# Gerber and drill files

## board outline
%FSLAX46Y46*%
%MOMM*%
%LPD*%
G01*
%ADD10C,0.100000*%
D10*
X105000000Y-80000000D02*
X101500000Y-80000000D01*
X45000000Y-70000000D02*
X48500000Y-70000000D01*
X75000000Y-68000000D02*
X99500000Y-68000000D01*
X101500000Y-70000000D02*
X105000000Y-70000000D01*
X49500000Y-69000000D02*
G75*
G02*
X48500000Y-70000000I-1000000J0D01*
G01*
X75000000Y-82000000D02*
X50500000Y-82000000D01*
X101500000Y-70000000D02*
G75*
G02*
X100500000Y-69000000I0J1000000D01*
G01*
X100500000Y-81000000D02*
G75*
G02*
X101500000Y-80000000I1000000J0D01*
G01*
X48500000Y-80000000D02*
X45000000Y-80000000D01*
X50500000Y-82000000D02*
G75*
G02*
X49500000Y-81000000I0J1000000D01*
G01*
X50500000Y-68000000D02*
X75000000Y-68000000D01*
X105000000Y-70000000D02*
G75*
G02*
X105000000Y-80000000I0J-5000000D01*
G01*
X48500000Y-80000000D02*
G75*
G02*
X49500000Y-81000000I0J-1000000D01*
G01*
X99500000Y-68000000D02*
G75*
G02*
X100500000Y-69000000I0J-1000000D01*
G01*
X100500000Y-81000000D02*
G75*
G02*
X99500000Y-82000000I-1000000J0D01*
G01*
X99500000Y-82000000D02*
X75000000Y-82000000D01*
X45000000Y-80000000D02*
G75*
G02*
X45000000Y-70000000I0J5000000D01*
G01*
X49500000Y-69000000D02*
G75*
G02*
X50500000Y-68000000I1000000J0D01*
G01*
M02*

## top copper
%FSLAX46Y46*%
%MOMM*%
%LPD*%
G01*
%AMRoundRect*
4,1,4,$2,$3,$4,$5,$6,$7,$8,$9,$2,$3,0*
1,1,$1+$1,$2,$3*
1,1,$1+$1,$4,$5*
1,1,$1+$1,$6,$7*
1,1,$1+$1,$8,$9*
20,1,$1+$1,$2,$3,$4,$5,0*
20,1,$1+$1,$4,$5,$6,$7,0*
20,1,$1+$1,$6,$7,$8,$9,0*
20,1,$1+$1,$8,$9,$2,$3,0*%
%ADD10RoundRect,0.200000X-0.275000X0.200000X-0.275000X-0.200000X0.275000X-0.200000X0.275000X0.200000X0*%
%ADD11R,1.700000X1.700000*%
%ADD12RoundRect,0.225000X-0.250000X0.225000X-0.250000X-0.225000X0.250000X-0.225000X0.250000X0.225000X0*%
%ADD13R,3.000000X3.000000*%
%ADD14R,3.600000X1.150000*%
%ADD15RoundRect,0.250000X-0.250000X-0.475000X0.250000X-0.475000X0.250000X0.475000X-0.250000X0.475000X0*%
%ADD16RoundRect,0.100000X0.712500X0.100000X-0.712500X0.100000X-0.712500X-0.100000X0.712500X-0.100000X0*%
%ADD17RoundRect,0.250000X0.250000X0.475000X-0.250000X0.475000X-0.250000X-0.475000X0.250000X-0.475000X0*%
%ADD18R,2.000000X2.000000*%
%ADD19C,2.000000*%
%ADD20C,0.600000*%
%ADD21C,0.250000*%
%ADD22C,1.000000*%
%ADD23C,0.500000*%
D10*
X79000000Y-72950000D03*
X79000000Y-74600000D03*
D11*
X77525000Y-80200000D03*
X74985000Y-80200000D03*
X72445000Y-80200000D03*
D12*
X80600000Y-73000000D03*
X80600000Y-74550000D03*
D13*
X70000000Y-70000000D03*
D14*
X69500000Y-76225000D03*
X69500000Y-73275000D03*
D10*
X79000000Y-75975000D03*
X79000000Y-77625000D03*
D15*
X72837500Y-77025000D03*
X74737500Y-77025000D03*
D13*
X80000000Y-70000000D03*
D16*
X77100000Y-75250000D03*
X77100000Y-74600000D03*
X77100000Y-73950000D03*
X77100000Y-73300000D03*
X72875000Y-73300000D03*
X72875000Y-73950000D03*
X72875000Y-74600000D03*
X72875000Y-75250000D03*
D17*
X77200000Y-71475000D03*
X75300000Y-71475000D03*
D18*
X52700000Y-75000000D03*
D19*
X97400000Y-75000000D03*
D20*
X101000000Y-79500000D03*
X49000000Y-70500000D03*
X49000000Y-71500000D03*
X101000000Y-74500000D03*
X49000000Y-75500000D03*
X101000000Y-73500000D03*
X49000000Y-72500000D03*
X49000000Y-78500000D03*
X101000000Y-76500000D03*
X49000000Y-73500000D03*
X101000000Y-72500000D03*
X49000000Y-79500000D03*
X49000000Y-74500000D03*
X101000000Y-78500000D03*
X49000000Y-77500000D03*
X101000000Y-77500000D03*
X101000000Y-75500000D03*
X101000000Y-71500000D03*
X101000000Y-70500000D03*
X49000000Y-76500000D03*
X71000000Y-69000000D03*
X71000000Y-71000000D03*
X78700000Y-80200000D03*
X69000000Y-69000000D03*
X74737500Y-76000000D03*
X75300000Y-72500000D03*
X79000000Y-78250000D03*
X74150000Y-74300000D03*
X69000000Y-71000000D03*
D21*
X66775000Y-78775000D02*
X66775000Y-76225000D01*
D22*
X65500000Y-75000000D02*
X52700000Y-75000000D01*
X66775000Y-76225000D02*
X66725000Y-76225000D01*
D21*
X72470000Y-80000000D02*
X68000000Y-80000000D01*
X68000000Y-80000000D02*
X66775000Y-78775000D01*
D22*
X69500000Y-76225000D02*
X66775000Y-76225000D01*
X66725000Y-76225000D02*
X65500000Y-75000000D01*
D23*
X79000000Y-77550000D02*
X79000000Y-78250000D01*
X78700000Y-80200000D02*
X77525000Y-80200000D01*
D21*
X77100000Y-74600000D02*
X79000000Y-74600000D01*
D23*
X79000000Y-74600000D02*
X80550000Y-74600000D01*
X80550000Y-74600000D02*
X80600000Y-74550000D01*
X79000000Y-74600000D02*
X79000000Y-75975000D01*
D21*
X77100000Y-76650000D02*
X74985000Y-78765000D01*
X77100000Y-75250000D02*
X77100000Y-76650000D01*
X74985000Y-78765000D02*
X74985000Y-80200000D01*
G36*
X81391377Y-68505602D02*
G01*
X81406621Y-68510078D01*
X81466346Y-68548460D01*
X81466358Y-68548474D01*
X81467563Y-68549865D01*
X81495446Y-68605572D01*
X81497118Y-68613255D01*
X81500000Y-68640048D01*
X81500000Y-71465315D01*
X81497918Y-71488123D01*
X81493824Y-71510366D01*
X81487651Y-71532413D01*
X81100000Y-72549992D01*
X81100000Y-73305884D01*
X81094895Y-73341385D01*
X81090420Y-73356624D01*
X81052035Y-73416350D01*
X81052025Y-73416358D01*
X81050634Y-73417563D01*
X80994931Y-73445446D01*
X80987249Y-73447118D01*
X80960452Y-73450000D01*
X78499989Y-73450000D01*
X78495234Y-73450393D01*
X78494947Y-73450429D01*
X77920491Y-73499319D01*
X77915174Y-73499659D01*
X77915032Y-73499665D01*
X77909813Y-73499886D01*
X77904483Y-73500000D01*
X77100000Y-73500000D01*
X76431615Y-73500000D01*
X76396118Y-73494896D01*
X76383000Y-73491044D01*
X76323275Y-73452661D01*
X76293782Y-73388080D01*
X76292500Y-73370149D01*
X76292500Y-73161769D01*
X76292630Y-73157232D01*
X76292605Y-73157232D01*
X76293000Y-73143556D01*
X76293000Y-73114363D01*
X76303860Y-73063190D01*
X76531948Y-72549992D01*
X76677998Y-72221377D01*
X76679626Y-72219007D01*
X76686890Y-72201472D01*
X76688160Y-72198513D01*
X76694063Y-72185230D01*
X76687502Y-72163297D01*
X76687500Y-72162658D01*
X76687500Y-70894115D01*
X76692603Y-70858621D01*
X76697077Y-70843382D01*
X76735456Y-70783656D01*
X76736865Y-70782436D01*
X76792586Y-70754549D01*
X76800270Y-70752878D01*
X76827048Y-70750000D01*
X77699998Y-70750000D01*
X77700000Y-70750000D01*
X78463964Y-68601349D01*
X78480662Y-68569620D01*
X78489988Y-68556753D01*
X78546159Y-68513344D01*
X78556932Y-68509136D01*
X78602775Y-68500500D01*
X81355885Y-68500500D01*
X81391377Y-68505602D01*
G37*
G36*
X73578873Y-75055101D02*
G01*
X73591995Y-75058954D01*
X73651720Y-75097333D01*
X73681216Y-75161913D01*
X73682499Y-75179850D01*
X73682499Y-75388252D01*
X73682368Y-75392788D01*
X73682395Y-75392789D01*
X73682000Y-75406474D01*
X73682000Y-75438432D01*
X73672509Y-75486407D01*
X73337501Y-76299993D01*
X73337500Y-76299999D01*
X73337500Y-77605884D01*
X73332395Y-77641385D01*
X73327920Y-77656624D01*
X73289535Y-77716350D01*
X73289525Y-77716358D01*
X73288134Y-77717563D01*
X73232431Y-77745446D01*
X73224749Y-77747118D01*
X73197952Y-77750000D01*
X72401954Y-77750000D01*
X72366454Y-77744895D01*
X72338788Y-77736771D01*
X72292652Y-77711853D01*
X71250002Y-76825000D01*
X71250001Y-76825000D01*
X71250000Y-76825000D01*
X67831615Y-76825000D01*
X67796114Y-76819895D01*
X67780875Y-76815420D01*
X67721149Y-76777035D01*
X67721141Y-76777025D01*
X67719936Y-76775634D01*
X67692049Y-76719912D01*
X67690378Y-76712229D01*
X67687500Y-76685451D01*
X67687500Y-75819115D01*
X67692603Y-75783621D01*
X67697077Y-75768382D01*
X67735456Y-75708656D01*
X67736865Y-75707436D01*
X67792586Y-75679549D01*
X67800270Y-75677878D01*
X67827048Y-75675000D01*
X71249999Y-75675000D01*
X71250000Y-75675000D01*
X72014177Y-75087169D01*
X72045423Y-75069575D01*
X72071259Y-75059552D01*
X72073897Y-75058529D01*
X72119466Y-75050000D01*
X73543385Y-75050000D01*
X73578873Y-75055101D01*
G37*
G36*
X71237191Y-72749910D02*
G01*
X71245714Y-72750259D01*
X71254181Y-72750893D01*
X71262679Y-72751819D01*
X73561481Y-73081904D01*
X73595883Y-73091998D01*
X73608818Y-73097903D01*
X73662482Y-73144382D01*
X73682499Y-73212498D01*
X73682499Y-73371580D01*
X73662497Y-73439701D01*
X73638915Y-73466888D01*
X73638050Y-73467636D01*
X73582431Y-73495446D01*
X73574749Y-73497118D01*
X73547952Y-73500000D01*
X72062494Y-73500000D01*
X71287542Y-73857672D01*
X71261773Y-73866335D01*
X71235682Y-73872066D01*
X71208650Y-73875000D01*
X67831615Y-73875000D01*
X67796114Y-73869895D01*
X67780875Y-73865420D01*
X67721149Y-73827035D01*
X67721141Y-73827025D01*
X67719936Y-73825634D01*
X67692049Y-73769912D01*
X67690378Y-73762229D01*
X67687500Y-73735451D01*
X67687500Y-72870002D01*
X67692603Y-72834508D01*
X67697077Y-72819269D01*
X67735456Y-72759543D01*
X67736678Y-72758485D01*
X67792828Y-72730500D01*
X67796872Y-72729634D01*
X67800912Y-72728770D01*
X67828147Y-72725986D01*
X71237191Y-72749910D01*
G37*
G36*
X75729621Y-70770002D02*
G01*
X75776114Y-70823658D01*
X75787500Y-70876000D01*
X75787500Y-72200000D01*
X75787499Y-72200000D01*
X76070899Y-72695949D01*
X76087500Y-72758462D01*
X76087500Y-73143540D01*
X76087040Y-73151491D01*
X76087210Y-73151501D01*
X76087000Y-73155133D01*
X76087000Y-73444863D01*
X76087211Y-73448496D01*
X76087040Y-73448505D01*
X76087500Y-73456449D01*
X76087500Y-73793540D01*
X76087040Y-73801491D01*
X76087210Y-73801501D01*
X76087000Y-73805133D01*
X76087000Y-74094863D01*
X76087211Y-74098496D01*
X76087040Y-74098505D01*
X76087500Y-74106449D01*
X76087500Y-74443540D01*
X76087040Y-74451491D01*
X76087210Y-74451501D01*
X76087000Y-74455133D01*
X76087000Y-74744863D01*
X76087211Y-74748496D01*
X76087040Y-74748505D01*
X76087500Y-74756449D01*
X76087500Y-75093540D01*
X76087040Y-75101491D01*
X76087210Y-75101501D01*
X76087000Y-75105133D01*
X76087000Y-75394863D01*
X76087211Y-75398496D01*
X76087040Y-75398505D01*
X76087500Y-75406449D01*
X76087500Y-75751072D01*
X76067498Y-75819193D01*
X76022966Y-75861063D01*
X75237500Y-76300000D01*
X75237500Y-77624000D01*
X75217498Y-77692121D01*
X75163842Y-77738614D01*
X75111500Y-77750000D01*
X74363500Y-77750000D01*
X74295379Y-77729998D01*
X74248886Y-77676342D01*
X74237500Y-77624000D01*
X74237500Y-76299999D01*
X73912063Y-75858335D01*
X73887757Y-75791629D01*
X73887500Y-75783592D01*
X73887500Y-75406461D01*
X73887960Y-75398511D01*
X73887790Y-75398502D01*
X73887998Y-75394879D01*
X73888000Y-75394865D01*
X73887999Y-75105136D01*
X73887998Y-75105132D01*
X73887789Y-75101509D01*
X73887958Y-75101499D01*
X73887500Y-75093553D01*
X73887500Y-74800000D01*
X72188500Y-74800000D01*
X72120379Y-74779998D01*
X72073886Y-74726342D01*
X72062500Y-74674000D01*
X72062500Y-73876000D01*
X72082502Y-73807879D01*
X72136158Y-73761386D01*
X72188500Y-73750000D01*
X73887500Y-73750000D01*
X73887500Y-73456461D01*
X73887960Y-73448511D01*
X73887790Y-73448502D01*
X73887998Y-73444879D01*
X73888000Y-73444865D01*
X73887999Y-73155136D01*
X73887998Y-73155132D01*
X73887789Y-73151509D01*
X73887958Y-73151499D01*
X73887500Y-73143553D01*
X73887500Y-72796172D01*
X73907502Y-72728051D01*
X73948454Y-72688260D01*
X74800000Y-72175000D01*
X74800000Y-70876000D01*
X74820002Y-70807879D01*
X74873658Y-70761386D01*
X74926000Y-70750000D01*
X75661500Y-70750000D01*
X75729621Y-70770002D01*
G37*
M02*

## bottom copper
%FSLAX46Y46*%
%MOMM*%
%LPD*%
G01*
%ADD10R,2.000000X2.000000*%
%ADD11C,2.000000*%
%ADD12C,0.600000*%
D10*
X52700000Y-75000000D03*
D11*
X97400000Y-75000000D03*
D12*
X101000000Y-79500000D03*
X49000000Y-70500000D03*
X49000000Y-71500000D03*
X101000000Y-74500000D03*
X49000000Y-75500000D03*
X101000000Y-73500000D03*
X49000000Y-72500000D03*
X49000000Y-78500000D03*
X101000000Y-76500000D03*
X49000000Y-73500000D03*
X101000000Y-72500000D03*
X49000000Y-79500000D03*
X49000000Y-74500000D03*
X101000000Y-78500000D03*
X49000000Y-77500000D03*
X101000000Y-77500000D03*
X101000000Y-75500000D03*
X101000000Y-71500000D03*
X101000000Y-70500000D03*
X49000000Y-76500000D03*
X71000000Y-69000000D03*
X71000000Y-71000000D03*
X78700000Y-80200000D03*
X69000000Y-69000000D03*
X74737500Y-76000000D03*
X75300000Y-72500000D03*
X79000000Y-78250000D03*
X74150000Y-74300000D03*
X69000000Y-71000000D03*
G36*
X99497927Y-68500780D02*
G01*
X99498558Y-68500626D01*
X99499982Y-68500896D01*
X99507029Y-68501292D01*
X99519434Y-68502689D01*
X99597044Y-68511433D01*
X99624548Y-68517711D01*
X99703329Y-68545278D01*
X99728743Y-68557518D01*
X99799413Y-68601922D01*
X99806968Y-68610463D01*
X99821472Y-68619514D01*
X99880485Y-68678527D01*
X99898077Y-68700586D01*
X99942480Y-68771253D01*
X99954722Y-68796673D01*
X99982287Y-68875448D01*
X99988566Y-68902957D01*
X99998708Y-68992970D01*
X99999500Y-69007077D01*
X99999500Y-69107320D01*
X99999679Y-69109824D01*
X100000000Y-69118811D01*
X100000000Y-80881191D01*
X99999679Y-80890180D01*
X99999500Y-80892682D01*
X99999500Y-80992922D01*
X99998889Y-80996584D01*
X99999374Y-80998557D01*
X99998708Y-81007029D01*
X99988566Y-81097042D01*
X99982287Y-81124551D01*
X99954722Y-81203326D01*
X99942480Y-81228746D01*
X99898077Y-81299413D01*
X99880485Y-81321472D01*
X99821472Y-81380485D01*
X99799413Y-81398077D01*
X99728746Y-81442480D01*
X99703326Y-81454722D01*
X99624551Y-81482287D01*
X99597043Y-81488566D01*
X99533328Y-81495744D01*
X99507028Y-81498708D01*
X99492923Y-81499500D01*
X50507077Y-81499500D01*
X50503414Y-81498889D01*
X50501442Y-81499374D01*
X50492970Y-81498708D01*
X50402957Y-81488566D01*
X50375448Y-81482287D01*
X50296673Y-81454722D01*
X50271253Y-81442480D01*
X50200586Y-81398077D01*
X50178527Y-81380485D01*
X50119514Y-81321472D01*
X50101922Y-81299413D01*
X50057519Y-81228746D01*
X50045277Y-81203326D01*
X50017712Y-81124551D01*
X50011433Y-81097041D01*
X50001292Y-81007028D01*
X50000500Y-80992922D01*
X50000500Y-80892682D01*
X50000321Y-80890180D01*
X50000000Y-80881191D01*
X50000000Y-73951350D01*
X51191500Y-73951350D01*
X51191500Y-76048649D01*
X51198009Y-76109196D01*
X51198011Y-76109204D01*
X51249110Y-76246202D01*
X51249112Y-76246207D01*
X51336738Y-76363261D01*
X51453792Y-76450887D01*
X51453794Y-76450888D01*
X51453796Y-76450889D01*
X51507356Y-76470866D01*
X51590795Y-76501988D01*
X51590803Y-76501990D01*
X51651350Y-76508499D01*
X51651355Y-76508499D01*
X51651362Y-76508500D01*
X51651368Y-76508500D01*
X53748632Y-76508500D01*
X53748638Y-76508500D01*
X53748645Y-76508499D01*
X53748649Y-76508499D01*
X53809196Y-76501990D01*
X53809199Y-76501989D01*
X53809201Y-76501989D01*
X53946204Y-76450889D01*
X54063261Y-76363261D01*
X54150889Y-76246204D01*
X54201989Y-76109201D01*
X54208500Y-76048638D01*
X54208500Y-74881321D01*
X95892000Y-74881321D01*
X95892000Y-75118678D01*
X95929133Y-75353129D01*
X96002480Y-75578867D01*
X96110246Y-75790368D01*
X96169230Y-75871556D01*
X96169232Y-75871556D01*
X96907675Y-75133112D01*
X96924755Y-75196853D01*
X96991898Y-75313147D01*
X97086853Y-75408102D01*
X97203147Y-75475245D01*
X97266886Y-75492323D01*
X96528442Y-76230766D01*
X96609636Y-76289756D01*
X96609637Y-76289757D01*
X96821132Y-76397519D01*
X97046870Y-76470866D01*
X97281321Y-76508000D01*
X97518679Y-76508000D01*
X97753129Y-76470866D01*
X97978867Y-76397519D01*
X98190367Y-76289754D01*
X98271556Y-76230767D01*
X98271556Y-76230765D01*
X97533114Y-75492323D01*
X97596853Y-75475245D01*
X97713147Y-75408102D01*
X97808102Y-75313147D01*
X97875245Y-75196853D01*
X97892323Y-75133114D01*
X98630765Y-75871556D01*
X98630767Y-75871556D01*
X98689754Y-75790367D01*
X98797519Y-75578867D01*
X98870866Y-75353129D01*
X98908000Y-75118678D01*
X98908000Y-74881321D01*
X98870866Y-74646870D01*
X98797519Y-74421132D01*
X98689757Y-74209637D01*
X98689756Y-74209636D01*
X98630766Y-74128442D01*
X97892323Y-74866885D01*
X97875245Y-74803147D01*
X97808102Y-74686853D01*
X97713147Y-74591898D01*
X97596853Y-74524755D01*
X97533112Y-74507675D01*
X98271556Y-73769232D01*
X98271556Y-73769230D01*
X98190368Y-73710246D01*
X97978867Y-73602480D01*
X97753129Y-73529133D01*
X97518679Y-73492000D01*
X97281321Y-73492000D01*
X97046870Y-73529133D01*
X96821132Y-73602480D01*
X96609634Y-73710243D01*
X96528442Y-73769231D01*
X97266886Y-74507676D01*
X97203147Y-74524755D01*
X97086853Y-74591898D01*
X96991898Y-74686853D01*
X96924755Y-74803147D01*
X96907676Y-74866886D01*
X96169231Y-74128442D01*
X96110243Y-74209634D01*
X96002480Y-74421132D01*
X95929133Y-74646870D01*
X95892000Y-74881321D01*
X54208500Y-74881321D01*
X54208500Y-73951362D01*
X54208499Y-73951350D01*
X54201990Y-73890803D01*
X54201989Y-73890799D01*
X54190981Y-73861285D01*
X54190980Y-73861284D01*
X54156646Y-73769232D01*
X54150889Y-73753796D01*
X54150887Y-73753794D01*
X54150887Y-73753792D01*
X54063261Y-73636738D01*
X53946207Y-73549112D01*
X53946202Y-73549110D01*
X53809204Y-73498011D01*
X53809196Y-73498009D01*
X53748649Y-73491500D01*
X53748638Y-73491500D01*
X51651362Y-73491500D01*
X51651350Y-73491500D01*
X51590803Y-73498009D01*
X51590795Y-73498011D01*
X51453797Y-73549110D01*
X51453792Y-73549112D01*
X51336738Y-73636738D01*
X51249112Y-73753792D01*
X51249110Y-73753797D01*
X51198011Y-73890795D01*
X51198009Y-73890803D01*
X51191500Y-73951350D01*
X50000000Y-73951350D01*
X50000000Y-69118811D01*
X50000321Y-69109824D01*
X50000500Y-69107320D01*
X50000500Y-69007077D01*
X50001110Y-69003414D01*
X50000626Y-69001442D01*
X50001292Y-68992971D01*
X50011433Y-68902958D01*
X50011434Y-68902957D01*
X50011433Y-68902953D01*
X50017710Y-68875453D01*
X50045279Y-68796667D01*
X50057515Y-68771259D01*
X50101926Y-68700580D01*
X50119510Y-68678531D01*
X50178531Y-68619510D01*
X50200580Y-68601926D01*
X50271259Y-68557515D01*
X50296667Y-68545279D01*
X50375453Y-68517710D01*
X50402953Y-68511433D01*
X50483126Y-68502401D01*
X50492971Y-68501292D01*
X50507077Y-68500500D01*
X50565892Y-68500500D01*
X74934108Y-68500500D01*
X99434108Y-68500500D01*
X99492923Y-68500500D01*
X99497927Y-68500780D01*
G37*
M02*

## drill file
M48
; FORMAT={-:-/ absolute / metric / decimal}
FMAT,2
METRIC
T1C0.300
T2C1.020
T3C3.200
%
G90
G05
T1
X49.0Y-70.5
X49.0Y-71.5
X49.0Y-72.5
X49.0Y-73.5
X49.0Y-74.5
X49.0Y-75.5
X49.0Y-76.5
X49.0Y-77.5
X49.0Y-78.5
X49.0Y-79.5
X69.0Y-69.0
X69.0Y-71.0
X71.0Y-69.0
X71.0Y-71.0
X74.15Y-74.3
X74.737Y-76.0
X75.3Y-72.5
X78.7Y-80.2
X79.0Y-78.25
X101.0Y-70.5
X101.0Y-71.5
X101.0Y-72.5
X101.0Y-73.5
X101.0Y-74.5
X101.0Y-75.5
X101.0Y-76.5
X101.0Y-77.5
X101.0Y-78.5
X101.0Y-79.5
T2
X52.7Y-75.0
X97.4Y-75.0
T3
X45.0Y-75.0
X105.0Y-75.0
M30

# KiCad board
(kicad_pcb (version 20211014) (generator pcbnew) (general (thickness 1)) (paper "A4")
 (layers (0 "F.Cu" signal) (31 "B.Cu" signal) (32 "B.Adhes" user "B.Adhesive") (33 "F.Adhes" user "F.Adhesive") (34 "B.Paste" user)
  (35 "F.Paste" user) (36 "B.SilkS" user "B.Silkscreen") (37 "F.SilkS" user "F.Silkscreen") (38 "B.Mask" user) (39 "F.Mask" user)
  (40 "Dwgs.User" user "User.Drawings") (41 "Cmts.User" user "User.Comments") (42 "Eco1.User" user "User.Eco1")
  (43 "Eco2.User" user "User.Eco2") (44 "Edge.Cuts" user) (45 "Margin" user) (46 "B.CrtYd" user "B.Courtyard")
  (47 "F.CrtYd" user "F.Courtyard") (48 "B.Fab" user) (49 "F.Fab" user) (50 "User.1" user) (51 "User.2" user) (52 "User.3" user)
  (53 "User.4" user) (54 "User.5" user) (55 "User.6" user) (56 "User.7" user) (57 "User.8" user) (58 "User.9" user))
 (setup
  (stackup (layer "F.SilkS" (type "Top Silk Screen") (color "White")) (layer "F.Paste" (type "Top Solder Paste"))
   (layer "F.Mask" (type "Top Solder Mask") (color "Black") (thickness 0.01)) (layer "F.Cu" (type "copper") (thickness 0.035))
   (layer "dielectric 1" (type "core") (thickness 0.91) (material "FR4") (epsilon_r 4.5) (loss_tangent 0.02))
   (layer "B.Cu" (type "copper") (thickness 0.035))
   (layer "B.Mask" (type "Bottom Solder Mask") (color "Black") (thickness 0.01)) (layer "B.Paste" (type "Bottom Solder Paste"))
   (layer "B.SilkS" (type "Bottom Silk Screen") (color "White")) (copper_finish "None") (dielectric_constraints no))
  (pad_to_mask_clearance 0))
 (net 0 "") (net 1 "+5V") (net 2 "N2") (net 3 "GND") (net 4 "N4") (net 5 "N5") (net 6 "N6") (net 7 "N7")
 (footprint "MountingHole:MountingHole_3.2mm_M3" (layer "F.Cu") (at 105 75)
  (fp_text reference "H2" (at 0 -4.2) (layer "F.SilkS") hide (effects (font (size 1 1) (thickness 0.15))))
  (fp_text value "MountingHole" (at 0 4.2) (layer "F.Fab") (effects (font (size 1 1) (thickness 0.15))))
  (pad "" np_thru_hole circle (at 0 0) (size 3.2 3.2) (drill 3.2) (layers *.Cu *.Mask)))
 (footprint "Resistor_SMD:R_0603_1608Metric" (layer "F.Cu") (at 79 73.775 -90)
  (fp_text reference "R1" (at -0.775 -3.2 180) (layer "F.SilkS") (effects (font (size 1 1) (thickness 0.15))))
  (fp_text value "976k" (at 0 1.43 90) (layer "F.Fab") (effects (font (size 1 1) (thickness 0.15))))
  (pad "1" smd roundrect (at -0.825 0 270) (size 0.8 0.95) (layers "F.Cu" "F.Paste" "F.Mask") (roundrect_rratio 0.25) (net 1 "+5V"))
  (pad "2" smd roundrect (at 0.825 0 270) (size 0.8 0.95) (layers "F.Cu" "F.Paste" "F.Mask") (roundrect_rratio 0.25) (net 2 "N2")))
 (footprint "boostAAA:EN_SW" (layer "F.Cu") (at 77.525 80.2 -90)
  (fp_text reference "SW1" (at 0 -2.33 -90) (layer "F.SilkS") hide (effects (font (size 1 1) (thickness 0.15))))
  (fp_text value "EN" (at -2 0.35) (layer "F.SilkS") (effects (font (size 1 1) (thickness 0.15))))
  (pad "1" smd rect (at 0 0 270) (size 1.7 1.7) (layers "F.Cu" "F.Mask") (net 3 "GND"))
  (pad "2" smd rect (at 0 2.54 270) (size 1.7 1.7) (layers "F.Cu" "F.Mask") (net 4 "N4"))
  (pad "3" smd rect (at 0 5.08 270) (size 1.7 1.7) (layers "F.Cu" "F.Mask") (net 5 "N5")))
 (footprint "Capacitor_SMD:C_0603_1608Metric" (layer "F.Cu") (at 80.6 73.775 -90)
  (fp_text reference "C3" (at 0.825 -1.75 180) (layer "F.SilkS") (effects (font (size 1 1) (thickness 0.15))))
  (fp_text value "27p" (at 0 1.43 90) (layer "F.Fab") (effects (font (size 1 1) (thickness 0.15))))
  (pad "1" smd roundrect (at -0.775 0 270) (size 0.9 0.95) (layers "F.Cu" "F.Paste" "F.Mask") (roundrect_rratio 0.25) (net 1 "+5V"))
  (pad "2" smd roundrect (at 0.775 0 270) (size 0.9 0.95) (layers "F.Cu" "F.Paste" "F.Mask") (roundrect_rratio 0.25) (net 2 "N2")))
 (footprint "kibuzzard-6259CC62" (layer "F.Cu") (at 59.5 75)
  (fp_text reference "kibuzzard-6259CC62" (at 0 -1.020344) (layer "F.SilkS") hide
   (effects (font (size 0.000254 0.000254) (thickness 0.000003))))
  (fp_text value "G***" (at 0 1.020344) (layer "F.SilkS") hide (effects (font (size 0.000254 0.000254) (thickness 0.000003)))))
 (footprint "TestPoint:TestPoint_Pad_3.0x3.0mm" (layer "F.Cu") (at 70 70)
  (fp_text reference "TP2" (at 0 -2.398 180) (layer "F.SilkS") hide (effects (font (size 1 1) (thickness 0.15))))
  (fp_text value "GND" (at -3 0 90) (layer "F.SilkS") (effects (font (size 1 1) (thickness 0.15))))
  (pad "1" smd rect (at 0 0) (size 3 3) (layers "F.Cu" "F.Mask") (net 3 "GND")))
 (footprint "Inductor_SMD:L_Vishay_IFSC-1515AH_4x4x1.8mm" (layer "F.Cu") (at 69.5 74.75 90)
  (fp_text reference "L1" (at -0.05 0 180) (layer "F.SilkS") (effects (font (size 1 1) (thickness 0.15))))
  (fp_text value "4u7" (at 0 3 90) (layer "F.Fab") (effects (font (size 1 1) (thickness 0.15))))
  (pad "1" smd rect (at -1.475 0 90) (size 1.15 3.6) (layers "F.Cu" "F.Paste" "F.Mask") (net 5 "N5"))
  (pad "2" smd rect (at 1.475 0 90) (size 1.15 3.6) (layers "F.Cu" "F.Paste" "F.Mask") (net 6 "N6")))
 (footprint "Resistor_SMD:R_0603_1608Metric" (layer "F.Cu") (at 79 76.8 -90)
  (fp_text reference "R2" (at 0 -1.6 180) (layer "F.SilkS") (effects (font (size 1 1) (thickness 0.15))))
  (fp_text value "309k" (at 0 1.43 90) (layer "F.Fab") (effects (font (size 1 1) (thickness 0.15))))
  (pad "1" smd roundrect (at -0.825 0 270) (size 0.8 0.95) (layers "F.Cu" "F.Paste" "F.Mask") (roundrect_rratio 0.25) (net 2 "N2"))
  (pad "2" smd roundrect (at 0.825 0 270) (size 0.8 0.95) (layers "F.Cu" "F.Paste" "F.Mask") (roundrect_rratio 0.25) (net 3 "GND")))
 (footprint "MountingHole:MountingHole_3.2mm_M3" (layer "F.Cu") (at 45 75)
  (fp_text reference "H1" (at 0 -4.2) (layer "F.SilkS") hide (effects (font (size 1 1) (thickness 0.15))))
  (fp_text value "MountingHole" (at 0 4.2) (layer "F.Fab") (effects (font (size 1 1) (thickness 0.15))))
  (pad "" np_thru_hole circle (at 0 0) (size 3.2 3.2) (drill 3.2) (layers *.Cu *.Mask)))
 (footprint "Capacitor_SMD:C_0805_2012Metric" (layer "F.Cu") (at 73.7875 77.025)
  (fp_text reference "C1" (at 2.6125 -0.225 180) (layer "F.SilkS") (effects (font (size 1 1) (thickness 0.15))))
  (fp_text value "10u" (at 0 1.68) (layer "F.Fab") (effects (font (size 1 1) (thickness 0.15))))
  (pad "1" smd roundrect (at -0.95 0) (size 1 1.45) (layers "F.Cu" "F.Paste" "F.Mask") (roundrect_rratio 0.25) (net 5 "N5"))
  (pad "2" smd roundrect (at 0.95 0) (size 1 1.45) (layers "F.Cu" "F.Paste" "F.Mask") (roundrect_rratio 0.25) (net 3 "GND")))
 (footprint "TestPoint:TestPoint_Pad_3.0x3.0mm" (layer "F.Cu") (at 80 70) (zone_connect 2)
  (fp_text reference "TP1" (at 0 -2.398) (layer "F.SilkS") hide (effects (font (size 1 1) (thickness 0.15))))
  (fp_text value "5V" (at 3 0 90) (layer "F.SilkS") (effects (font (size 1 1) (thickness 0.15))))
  (pad "1" smd rect (at 0 0) (size 3 3) (layers "F.Cu" "F.Mask") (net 1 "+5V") (zone_connect 2)))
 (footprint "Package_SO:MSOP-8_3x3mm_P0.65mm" (layer "F.Cu") (at 74.9875 74.275 180)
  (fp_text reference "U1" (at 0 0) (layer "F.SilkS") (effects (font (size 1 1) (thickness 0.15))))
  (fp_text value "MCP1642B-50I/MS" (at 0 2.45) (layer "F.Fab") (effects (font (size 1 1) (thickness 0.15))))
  (pad "1" smd roundrect (at -2.1125 -0.975 180) (size 1.625 0.4) (layers "F.Cu" "F.Paste" "F.Mask") (roundrect_rratio 0.25) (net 4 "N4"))
  (pad "2" smd roundrect (at -2.1125 -0.325 180) (size 1.625 0.4) (layers "F.Cu" "F.Paste" "F.Mask") (roundrect_rratio 0.25) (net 2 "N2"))
  (pad "3" smd roundrect (at -2.1125 0.325 180) (size 1.625 0.4) (layers "F.Cu" "F.Paste" "F.Mask") (roundrect_rratio 0.25) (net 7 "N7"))
  (pad "4" smd roundrect (at -2.1125 0.975 180) (size 1.625 0.4) (layers "F.Cu" "F.Paste" "F.Mask") (roundrect_rratio 0.25) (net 1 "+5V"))
  (pad "5" smd roundrect (at 2.1125 0.975 180) (size 1.625 0.4) (layers "F.Cu" "F.Paste" "F.Mask") (roundrect_rratio 0.25) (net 6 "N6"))
  (pad "6" smd roundrect (at 2.1125 0.325 180) (size 1.625 0.4) (layers "F.Cu" "F.Paste" "F.Mask") (roundrect_rratio 0.25) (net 3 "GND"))
  (pad "7" smd roundrect (at 2.1125 -0.325 180) (size 1.625 0.4) (layers "F.Cu" "F.Paste" "F.Mask") (roundrect_rratio 0.25) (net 3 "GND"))
  (pad "8" smd roundrect (at 2.1125 -0.975 180) (size 1.625 0.4) (layers "F.Cu" "F.Paste" "F.Mask") (roundrect_rratio 0.25) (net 5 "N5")))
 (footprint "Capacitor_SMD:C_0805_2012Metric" (layer "F.Cu") (at 76.25 71.475 180)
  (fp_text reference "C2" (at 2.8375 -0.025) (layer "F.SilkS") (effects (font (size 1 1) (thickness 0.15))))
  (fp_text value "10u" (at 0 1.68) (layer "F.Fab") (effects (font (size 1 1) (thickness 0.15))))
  (pad "1" smd roundrect (at -0.95 0 180) (size 1 1.45) (layers "F.Cu" "F.Paste" "F.Mask") (roundrect_rratio 0.25) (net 1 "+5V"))
  (pad "2" smd roundrect (at 0.95 0 180) (size 1 1.45) (layers "F.Cu" "F.Paste" "F.Mask") (roundrect_rratio 0.25) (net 3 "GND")))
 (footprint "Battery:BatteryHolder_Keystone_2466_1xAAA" (layer "B.Cu") (at 52.7 75)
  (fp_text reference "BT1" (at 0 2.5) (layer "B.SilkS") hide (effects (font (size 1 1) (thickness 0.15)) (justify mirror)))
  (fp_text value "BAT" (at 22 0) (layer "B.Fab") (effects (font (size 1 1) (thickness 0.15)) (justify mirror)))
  (pad "1" thru_hole rect (at 0 0) (size 2 2) (drill 1.02) (layers *.Cu *.Mask) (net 5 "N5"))
  (pad "2" thru_hole circle (at 44.7 0) (size 2 2) (drill 1.02) (layers *.Cu *.Mask) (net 3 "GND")))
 (gr_line (start 105 80) (end 101.5 80) (layer "Edge.Cuts") (width 0.1))
 (gr_line (start 45 70) (end 48.5 70) (layer "Edge.Cuts") (width 0.1))
 (gr_line (start 75 68) (end 99.5 68) (layer "Edge.Cuts") (width 0.1))
 (gr_line (start 101.5 70) (end 105 70) (layer "Edge.Cuts") (width 0.1))
 (gr_arc (start 49.5 69) (mid 49.207107 69.707107) (end 48.5 70) (layer "Edge.Cuts") (width 0.1))
 (gr_line (start 75 82) (end 50.5 82) (layer "Edge.Cuts") (width 0.1))
 (gr_arc (start 101.5 70) (mid 100.792893 69.707107) (end 100.5 69) (layer "Edge.Cuts") (width 0.1))
 (gr_arc (start 100.5 81) (mid 100.792893 80.292893) (end 101.5 80) (layer "Edge.Cuts") (width 0.1))
 (gr_line (start 48.5 80) (end 45 80) (layer "Edge.Cuts") (width 0.1))
 (gr_arc (start 50.5 82) (mid 49.792893 81.707107) (end 49.5 81) (layer "Edge.Cuts") (width 0.1))
 (gr_line (start 50.5 68) (end 75 68) (layer "Edge.Cuts") (width 0.1))
 (gr_arc (start 105 70) (mid 110 75) (end 105 80) (layer "Edge.Cuts") (width 0.1))
 (gr_arc (start 48.5 80) (mid 49.207107 80.292893) (end 49.5 81) (layer "Edge.Cuts") (width 0.1))
 (gr_arc (start 99.5 68) (mid 100.207107 68.292893) (end 100.5 69) (layer "Edge.Cuts") (width 0.1))
 (gr_arc (start 100.5 81) (mid 100.207107 81.707107) (end 99.5 82) (layer "Edge.Cuts") (width 0.1))
 (gr_line (start 99.5 82) (end 75 82) (layer "Edge.Cuts") (width 0.1))
 (gr_arc (start 45 80) (mid 40 75) (end 45 70) (layer "Edge.Cuts") (width 0.1))
 (gr_arc (start 49.5 69) (mid 49.792893 68.292893) (end 50.5 68) (layer "Edge.Cuts") (width 0.1))
 (via (at 101 79.5) (size 0.6) (drill 0.3) (layers "F.Cu" "B.Cu") (free) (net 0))
 (via (at 49 70.5) (size 0.6) (drill 0.3) (layers "F.Cu" "B.Cu") (free) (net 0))
 (via (at 49 71.5) (size 0.6) (drill 0.3) (layers "F.Cu" "B.Cu") (free) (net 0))
 (via (at 101 74.5) (size 0.6) (drill 0.3) (layers "F.Cu" "B.Cu") (free) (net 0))
 (via (at 49 75.5) (size 0.6) (drill 0.3) (layers "F.Cu" "B.Cu") (free) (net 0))
 (via (at 101 73.5) (size 0.6) (drill 0.3) (layers "F.Cu" "B.Cu") (free) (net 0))
 (via (at 49 72.5) (size 0.6) (drill 0.3) (layers "F.Cu" "B.Cu") (free) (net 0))
 (via (at 49 78.5) (size 0.6) (drill 0.3) (layers "F.Cu" "B.Cu") (free) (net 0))
 (via (at 101 76.5) (size 0.6) (drill 0.3) (layers "F.Cu" "B.Cu") (free) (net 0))
 (via (at 49 73.5) (size 0.6) (drill 0.3) (layers "F.Cu" "B.Cu") (free) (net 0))
 (via (at 101 72.5) (size 0.6) (drill 0.3) (layers "F.Cu" "B.Cu") (free) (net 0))
 (via (at 49 79.5) (size 0.6) (drill 0.3) (layers "F.Cu" "B.Cu") (free) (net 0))
 (via (at 49 74.5) (size 0.6) (drill 0.3) (layers "F.Cu" "B.Cu") (free) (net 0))
 (via (at 101 78.5) (size 0.6) (drill 0.3) (layers "F.Cu" "B.Cu") (free) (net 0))
 (via (at 49 77.5) (size 0.6) (drill 0.3) (layers "F.Cu" "B.Cu") (free) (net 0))
 (via (at 101 77.5) (size 0.6) (drill 0.3) (layers "F.Cu" "B.Cu") (free) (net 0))
 (via (at 101 75.5) (size 0.6) (drill 0.3) (layers "F.Cu" "B.Cu") (free) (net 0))
 (via (at 101 71.5) (size 0.6) (drill 0.3) (layers "F.Cu" "B.Cu") (free) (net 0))
 (via (at 101 70.5) (size 0.6) (drill 0.3) (layers "F.Cu" "B.Cu") (free) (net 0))
 (via (at 49 76.5) (size 0.6) (drill 0.3) (layers "F.Cu" "B.Cu") (free) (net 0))
 (segment (start 66.775 78.775) (end 66.775 76.225) (width 0.25) (layer "F.Cu") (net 5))
 (segment (start 65.5 75) (end 52.7 75) (width 1) (layer "F.Cu") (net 5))
 (segment (start 66.775 76.225) (end 66.725 76.225) (width 1) (layer "F.Cu") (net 5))
 (segment (start 72.47 80) (end 68 80) (width 0.25) (layer "F.Cu") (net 5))
 (segment (start 68 80) (end 66.775 78.775) (width 0.25) (layer "F.Cu") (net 5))
 (segment (start 69.5 76.225) (end 66.775 76.225) (width 1) (layer "F.Cu") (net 5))
 (segment (start 66.725 76.225) (end 65.5 75) (width 1) (layer "F.Cu") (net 5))
 (segment (start 79 77.55) (end 79 78.25) (width 0.5) (layer "F.Cu") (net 3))
 (segment (start 78.7 80.2) (end 77.525 80.2) (width 0.5) (layer "F.Cu") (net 3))
 (via (at 71 69) (size 0.6) (drill 0.3) (layers "F.Cu" "B.Cu") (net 3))
 (via (at 71 71) (size 0.6) (drill 0.3) (layers "F.Cu" "B.Cu") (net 3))
 (via (at 78.7 80.2) (size 0.6) (drill 0.3) (layers "F.Cu" "B.Cu") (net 3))
 (via (at 69 69) (size 0.6) (drill 0.3) (layers "F.Cu" "B.Cu") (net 3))
 (via (at 74.7375 76) (size 0.6) (drill 0.3) (layers "F.Cu" "B.Cu") (free) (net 3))
 (via (at 75.3 72.5) (size 0.6) (drill 0.3) (layers "F.Cu" "B.Cu") (free) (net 3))
 (via (at 79 78.25) (size 0.6) (drill 0.3) (layers "F.Cu" "B.Cu") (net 3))
 (via (at 74.15 74.3) (size 0.6) (drill 0.3) (layers "F.Cu" "B.Cu") (free) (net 3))
 (via (at 69 71) (size 0.6) (drill 0.3) (layers "F.Cu" "B.Cu") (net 3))
 (segment (start 77.1 74.6) (end 79 74.6) (width 0.25) (layer "F.Cu") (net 2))
 (segment (start 79 74.6) (end 80.55 74.6) (width 0.5) (layer "F.Cu") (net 2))
 (segment (start 80.55 74.6) (end 80.6 74.55) (width 0.5) (layer "F.Cu") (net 2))
 (segment (start 79 74.6) (end 79 75.975) (width 0.5) (layer "F.Cu") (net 2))
 (segment (start 77.1 76.65) (end 74.985 78.765) (width 0.25) (layer "F.Cu") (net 4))
 (segment (start 77.1 75.25) (end 77.1 76.65) (width 0.25) (layer "F.Cu") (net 4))
 (segment (start 74.985 78.765) (end 74.985 80.2) (width 0.25) (layer "F.Cu") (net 4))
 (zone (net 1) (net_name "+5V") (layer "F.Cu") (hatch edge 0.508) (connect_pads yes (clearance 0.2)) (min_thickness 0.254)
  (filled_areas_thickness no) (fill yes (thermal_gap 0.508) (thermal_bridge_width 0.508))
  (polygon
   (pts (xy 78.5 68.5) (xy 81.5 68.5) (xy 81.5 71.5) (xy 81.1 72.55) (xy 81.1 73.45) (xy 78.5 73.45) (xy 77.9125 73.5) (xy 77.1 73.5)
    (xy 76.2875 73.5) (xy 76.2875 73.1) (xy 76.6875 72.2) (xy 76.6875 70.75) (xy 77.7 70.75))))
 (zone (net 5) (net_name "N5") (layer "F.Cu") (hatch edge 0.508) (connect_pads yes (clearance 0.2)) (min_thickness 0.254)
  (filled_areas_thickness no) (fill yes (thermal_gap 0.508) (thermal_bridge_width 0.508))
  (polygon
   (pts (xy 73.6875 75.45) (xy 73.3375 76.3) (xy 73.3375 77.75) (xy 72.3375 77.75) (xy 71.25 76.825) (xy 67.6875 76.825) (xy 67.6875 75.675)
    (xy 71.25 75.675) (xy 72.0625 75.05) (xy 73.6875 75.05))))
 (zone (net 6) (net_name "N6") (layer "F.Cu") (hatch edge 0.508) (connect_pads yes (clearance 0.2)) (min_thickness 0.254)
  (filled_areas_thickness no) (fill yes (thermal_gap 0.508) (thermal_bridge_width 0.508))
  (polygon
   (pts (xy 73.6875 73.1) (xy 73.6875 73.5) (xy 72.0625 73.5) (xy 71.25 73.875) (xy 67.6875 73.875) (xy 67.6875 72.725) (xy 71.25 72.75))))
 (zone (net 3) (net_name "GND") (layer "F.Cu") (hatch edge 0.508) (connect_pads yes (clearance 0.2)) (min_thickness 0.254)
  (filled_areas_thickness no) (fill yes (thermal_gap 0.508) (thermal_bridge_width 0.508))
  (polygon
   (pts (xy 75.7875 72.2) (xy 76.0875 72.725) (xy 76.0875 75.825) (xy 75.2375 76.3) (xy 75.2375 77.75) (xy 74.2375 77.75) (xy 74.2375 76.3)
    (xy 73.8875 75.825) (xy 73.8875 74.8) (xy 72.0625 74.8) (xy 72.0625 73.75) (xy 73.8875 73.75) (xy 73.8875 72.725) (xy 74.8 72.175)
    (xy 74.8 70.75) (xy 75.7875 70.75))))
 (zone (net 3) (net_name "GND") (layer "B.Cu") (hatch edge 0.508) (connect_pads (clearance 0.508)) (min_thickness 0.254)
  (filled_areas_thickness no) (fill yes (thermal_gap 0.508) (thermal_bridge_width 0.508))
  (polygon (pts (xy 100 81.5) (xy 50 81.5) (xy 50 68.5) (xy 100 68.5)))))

